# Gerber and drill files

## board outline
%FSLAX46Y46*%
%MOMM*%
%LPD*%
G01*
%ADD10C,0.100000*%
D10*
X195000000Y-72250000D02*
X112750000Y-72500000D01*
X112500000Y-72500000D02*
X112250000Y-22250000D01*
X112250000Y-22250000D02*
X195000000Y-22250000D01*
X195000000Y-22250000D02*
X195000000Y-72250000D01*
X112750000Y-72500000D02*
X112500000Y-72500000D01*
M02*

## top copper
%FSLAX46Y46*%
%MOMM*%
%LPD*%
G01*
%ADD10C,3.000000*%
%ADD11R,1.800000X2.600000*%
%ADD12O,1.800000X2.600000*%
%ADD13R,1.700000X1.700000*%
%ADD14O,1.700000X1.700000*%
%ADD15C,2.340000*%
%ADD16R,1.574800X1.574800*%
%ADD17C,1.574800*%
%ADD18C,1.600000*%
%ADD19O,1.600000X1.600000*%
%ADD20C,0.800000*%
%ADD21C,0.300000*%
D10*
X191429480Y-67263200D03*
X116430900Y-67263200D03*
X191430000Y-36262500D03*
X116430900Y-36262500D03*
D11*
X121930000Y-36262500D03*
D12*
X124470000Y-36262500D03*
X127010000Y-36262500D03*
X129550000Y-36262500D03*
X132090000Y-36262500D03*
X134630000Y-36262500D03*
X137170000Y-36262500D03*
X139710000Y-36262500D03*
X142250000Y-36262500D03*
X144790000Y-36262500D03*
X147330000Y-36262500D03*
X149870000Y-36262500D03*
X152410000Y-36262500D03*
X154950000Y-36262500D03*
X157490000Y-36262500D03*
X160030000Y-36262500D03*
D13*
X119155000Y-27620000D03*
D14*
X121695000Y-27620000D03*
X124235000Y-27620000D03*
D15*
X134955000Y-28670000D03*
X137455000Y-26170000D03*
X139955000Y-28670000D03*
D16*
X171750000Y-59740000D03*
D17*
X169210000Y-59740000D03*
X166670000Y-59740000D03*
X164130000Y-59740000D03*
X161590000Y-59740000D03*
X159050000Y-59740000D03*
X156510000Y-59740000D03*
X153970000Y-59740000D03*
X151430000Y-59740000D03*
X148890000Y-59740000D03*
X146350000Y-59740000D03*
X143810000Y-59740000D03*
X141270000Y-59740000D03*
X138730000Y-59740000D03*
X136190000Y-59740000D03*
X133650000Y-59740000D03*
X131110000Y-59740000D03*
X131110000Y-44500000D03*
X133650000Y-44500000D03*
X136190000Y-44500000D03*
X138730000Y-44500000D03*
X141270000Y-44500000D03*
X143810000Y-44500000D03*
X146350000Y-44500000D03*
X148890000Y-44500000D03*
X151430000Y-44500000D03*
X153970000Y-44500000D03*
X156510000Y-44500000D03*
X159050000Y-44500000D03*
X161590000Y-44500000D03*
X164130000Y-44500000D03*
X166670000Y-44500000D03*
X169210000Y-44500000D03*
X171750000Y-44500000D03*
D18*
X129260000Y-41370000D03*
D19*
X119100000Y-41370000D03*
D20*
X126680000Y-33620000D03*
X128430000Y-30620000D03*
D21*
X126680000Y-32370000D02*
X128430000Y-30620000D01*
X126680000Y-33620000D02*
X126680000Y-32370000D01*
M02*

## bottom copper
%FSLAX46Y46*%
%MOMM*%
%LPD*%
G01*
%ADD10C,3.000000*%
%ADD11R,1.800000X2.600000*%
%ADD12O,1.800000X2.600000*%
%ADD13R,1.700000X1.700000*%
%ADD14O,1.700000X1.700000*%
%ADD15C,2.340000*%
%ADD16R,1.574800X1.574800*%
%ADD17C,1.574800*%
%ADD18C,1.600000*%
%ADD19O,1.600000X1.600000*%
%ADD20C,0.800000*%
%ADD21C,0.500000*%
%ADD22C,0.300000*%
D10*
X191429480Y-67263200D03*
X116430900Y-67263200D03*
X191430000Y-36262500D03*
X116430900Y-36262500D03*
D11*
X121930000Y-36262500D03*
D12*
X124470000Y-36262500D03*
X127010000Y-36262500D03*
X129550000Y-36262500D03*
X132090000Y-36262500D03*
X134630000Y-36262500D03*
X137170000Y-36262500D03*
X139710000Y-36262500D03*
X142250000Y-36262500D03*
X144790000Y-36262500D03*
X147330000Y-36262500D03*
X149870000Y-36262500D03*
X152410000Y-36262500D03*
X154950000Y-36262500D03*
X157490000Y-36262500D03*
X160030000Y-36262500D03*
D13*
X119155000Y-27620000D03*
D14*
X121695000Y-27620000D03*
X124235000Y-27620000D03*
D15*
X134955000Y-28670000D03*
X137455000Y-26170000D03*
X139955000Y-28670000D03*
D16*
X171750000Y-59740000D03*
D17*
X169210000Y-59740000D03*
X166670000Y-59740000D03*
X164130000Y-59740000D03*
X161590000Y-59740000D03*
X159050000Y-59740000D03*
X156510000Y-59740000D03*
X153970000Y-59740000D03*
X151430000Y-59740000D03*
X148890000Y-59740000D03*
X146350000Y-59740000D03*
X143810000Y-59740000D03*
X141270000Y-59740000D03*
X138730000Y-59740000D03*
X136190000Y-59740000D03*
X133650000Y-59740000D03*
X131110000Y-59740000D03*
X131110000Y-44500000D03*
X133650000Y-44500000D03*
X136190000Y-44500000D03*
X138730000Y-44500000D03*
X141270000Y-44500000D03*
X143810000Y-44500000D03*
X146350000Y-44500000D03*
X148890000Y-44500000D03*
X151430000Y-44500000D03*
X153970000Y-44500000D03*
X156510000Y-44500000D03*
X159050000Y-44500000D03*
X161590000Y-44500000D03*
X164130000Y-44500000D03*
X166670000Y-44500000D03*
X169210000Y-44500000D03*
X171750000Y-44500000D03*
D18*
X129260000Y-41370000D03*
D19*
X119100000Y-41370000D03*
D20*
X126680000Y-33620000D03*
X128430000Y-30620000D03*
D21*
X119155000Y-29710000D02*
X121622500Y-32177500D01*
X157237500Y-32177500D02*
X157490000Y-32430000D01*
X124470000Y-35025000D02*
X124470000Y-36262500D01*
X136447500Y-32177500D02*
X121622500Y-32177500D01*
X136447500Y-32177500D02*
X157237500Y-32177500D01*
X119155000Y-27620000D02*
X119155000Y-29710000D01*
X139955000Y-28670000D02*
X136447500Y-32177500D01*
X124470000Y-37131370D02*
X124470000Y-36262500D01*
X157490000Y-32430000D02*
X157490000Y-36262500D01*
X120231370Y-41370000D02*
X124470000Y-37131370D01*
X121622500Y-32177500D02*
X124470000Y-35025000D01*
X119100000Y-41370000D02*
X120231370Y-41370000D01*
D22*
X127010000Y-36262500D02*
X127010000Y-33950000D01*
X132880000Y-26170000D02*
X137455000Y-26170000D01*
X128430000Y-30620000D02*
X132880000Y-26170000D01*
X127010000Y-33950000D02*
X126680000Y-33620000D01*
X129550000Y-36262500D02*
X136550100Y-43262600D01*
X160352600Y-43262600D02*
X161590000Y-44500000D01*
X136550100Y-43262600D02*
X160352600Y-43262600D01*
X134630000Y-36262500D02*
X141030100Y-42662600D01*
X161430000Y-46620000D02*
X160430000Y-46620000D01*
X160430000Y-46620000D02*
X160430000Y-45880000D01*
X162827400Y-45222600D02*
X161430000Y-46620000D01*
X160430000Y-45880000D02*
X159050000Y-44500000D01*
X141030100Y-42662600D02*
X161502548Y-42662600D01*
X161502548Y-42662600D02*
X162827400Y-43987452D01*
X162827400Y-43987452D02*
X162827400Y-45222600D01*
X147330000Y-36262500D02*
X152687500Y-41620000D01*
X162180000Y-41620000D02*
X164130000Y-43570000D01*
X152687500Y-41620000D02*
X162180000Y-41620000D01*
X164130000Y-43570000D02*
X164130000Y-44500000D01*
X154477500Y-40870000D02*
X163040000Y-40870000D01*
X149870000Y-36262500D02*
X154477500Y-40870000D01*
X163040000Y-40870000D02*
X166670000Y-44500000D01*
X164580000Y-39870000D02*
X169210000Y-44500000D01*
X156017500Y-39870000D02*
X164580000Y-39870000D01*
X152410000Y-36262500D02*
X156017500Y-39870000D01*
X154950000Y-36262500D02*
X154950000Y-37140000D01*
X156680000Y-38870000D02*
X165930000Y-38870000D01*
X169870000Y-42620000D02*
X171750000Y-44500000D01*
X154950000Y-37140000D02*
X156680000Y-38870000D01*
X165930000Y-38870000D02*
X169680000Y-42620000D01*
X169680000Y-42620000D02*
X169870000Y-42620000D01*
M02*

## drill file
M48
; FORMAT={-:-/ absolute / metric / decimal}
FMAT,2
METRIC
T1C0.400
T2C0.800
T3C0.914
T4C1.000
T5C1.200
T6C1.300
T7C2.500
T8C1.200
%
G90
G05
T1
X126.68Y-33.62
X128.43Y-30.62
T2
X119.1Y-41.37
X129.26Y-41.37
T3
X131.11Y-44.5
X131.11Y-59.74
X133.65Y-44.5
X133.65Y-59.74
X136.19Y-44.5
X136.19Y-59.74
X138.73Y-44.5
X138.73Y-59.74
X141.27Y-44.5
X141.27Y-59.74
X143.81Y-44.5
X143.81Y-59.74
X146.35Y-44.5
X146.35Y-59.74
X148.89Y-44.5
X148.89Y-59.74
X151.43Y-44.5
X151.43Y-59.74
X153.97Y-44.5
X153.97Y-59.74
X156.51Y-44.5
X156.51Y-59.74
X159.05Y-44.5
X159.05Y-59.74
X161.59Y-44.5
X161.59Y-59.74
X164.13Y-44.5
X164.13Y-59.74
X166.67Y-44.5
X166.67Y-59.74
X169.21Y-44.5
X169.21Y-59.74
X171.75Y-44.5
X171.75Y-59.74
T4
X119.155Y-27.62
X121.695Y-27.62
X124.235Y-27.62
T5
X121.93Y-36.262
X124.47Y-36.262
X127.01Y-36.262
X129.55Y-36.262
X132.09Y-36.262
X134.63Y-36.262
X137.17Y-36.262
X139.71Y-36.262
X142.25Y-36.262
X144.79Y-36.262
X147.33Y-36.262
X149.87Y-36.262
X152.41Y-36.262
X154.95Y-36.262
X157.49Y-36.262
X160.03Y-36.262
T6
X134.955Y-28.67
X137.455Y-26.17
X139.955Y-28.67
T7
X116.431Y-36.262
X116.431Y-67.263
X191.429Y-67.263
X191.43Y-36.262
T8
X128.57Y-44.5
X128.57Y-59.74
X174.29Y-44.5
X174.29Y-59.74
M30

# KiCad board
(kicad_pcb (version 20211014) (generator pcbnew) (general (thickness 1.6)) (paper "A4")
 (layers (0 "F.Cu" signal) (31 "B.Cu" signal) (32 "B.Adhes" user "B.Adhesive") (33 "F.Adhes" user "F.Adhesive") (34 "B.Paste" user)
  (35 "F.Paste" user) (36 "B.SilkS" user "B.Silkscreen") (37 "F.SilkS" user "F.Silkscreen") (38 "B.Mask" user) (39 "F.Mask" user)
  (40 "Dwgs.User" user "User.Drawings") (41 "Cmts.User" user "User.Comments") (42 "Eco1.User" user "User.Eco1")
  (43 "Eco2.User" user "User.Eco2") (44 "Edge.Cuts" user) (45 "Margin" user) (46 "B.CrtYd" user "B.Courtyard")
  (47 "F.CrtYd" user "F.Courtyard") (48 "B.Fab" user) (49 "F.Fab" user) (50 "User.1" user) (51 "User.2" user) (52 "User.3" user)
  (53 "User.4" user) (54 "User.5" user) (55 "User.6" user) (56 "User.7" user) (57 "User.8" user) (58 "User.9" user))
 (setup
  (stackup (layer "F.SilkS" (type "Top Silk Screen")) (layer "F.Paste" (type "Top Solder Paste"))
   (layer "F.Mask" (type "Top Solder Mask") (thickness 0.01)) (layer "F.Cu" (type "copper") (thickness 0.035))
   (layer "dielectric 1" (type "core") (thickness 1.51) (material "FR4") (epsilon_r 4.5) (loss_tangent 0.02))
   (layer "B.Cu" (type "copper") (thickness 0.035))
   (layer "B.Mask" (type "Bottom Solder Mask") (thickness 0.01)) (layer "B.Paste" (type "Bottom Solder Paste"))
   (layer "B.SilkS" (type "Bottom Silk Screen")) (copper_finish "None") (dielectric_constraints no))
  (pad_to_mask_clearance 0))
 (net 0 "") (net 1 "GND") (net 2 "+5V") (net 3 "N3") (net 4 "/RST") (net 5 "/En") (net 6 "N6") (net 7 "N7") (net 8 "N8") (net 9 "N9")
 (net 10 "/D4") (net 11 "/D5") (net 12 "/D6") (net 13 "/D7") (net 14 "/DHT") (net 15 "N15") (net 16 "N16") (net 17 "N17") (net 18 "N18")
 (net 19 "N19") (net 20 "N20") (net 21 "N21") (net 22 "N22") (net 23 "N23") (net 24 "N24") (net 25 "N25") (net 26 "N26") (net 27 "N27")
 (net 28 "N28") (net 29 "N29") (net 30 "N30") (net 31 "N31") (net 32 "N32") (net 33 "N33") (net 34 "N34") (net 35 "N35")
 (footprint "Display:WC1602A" (layer "F.Cu") (at 121.93 36.2625)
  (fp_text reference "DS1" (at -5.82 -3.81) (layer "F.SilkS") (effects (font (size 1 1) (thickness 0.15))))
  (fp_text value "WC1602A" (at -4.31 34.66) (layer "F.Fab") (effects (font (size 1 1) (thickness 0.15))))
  (pad "" thru_hole circle (at 69.49948 31.0007) (size 3 3) (drill 2.5) (layers *.Cu *.Mask))
  (pad "" thru_hole circle (at -5.4991 31.0007) (size 3 3) (drill 2.5) (layers *.Cu *.Mask))
  (pad "" thru_hole circle (at 69.5 0) (size 3 3) (drill 2.5) (layers *.Cu *.Mask))
  (pad "" thru_hole circle (at -5.4991 0) (size 3 3) (drill 2.5) (layers *.Cu *.Mask))
  (pad "1" thru_hole rect (at 0 0) (size 1.8 2.6) (drill 1.2) (layers *.Cu *.Mask) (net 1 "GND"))
  (pad "2" thru_hole oval (at 2.54 0) (size 1.8 2.6) (drill 1.2) (layers *.Cu *.Mask) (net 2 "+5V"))
  (pad "3" thru_hole oval (at 5.08 0) (size 1.8 2.6) (drill 1.2) (layers *.Cu *.Mask) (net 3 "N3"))
  (pad "4" thru_hole oval (at 7.62 0) (size 1.8 2.6) (drill 1.2) (layers *.Cu *.Mask) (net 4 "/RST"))
  (pad "5" thru_hole oval (at 10.16 0) (size 1.8 2.6) (drill 1.2) (layers *.Cu *.Mask) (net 1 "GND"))
  (pad "6" thru_hole oval (at 12.7 0) (size 1.8 2.6) (drill 1.2) (layers *.Cu *.Mask) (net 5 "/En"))
  (pad "7" thru_hole oval (at 15.24 0) (size 1.8 2.6) (drill 1.2) (layers *.Cu *.Mask) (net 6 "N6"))
  (pad "8" thru_hole oval (at 17.78 0) (size 1.8 2.6) (drill 1.2) (layers *.Cu *.Mask) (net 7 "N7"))
  (pad "9" thru_hole oval (at 20.32 0) (size 1.8 2.6) (drill 1.2) (layers *.Cu *.Mask) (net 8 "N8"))
  (pad "10" thru_hole oval (at 22.86 0) (size 1.8 2.6) (drill 1.2) (layers *.Cu *.Mask) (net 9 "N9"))
  (pad "11" thru_hole oval (at 25.4 0) (size 1.8 2.6) (drill 1.2) (layers *.Cu *.Mask) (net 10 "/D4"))
  (pad "12" thru_hole oval (at 27.94 0) (size 1.8 2.6) (drill 1.2) (layers *.Cu *.Mask) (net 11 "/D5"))
  (pad "13" thru_hole oval (at 30.48 0) (size 1.8 2.6) (drill 1.2) (layers *.Cu *.Mask) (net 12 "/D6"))
  (pad "14" thru_hole oval (at 33.02 0) (size 1.8 2.6) (drill 1.2) (layers *.Cu *.Mask) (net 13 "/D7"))
  (pad "15" thru_hole oval (at 35.56 0) (size 1.8 2.6) (drill 1.2) (layers *.Cu *.Mask) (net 2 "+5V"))
  (pad "16" thru_hole oval (at 38.1 0) (size 1.8 2.6) (drill 1.2) (layers *.Cu *.Mask) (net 1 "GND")))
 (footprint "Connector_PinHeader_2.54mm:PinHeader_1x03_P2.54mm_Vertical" (layer "F.Cu") (at 119.155 27.62 90)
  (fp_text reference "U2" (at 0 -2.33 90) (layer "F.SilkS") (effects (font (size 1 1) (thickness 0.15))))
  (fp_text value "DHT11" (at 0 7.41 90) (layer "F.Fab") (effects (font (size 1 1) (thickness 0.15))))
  (pad "1" thru_hole rect (at 0 0 90) (size 1.7 1.7) (drill 1) (layers *.Cu *.Mask) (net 2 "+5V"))
  (pad "2" thru_hole oval (at 0 2.54 90) (size 1.7 1.7) (drill 1) (layers *.Cu *.Mask) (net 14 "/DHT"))
  (pad "3" thru_hole oval (at 0 5.08 90) (size 1.7 1.7) (drill 1) (layers *.Cu *.Mask) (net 1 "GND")))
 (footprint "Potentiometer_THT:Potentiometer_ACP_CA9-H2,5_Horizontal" (layer "F.Cu") (at 134.955 28.67 90)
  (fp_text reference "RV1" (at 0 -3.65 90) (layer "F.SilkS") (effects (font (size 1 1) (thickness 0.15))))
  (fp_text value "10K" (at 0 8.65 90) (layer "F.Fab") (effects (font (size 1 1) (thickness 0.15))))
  (pad "1" thru_hole circle (at 0 0 90) (size 2.34 2.34) (drill 1.3) (layers *.Cu *.Mask) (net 1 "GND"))
  (pad "2" thru_hole circle (at 2.5 2.5 90) (size 2.34 2.34) (drill 1.3) (layers *.Cu *.Mask) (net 3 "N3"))
  (pad "3" thru_hole circle (at 0 5 90) (size 2.34 2.34) (drill 1.3) (layers *.Cu *.Mask) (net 2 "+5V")))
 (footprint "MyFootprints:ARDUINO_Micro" (layer "B.Cu") (at 151.43 52.12 90)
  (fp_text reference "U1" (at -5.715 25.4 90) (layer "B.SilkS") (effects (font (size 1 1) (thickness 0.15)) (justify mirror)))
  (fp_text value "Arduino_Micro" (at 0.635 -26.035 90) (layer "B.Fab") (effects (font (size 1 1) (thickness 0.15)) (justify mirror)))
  (pad "" np_thru_hole circle (at -7.62 -22.86 90) (size 1.2 1.2) (drill 1.2) (layers *.Cu *.Mask))
  (pad "" np_thru_hole circle (at 7.62 22.86 90) (size 1.2 1.2) (drill 1.2) (layers *.Cu *.Mask))
  (pad "" np_thru_hole circle (at -7.62 22.86 90) (size 1.2 1.2) (drill 1.2) (layers *.Cu *.Mask))
  (pad "" np_thru_hole circle (at 7.62 -22.86 90) (size 1.2 1.2) (drill 1.2) (layers *.Cu *.Mask))
  (pad "1" thru_hole rect (at -7.62 20.32 90) (size 1.5748 1.5748) (drill 0.9144) (layers *.Cu *.Mask) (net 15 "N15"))
  (pad "2" thru_hole circle (at -7.62 17.78 90) (size 1.5748 1.5748) (drill 0.9144) (layers *.Cu *.Mask) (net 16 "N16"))
  (pad "3" thru_hole circle (at -7.62 15.24 90) (size 1.5748 1.5748) (drill 0.9144) (layers *.Cu *.Mask) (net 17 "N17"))
  (pad "4" thru_hole circle (at -7.62 12.7 90) (size 1.5748 1.5748) (drill 0.9144) (layers *.Cu *.Mask) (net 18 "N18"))
  (pad "5" thru_hole circle (at -7.62 10.16 90) (size 1.5748 1.5748) (drill 0.9144) (layers *.Cu *.Mask) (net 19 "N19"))
  (pad "6" thru_hole circle (at -7.62 7.62 90) (size 1.5748 1.5748) (drill 0.9144) (layers *.Cu *.Mask) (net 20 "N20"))
  (pad "7" thru_hole circle (at -7.62 5.08 90) (size 1.5748 1.5748) (drill 0.9144) (layers *.Cu *.Mask) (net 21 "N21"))
  (pad "8" thru_hole circle (at -7.62 2.54 90) (size 1.5748 1.5748) (drill 0.9144) (layers *.Cu *.Mask) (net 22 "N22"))
  (pad "9" thru_hole circle (at -7.62 0 90) (size 1.5748 1.5748) (drill 0.9144) (layers *.Cu *.Mask) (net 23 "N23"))
  (pad "10" thru_hole circle (at -7.62 -2.54 90) (size 1.5748 1.5748) (drill 0.9144) (layers *.Cu *.Mask))
  (pad "11" thru_hole circle (at -7.62 -5.08 90) (size 1.5748 1.5748) (drill 0.9144) (layers *.Cu *.Mask))
  (pad "12" thru_hole circle (at -7.62 -7.62 90) (size 1.5748 1.5748) (drill 0.9144) (layers *.Cu *.Mask) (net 2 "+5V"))
  (pad "13" thru_hole circle (at -7.62 -10.16 90) (size 1.5748 1.5748) (drill 0.9144) (layers *.Cu *.Mask) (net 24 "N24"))
  (pad "14" thru_hole circle (at -7.62 -12.7 90) (size 1.5748 1.5748) (drill 0.9144) (layers *.Cu *.Mask) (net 1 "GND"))
  (pad "15" thru_hole circle (at -7.62 -15.24 90) (size 1.5748 1.5748) (drill 0.9144) (layers *.Cu *.Mask) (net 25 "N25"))
  (pad "16" thru_hole circle (at -7.62 -17.78 90) (size 1.5748 1.5748) (drill 0.9144) (layers *.Cu *.Mask) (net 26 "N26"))
  (pad "17" thru_hole circle (at -7.62 -20.32 90) (size 1.5748 1.5748) (drill 0.9144) (layers *.Cu *.Mask) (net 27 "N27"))
  (pad "18" thru_hole circle (at 7.62 -20.32 90) (size 1.5748 1.5748) (drill 0.9144) (layers *.Cu *.Mask) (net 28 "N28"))
  (pad "19" thru_hole circle (at 7.62 -17.78 90) (size 1.5748 1.5748) (drill 0.9144) (layers *.Cu *.Mask) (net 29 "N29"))
  (pad "20" thru_hole circle (at 7.62 -15.24 90) (size 1.5748 1.5748) (drill 0.9144) (layers *.Cu *.Mask) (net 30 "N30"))
  (pad "21" thru_hole circle (at 7.62 -12.7 90) (size 1.5748 1.5748) (drill 0.9144) (layers *.Cu *.Mask) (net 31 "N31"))
  (pad "22" thru_hole circle (at 7.62 -10.16 90) (size 1.5748 1.5748) (drill 0.9144) (layers *.Cu *.Mask))
  (pad "23" thru_hole circle (at 7.62 -7.62 90) (size 1.5748 1.5748) (drill 0.9144) (layers *.Cu *.Mask) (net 1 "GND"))
  (pad "24" thru_hole circle (at 7.62 -5.08 90) (size 1.5748 1.5748) (drill 0.9144) (layers *.Cu *.Mask) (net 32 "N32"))
  (pad "25" thru_hole circle (at 7.62 -2.54 90) (size 1.5748 1.5748) (drill 0.9144) (layers *.Cu *.Mask) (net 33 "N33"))
  (pad "26" thru_hole circle (at 7.62 0 90) (size 1.5748 1.5748) (drill 0.9144) (layers *.Cu *.Mask) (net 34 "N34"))
  (pad "27" thru_hole circle (at 7.62 2.54 90) (size 1.5748 1.5748) (drill 0.9144) (layers *.Cu *.Mask) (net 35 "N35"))
  (pad "28" thru_hole circle (at 7.62 5.08 90) (size 1.5748 1.5748) (drill 0.9144) (layers *.Cu *.Mask) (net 14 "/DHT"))
  (pad "29" thru_hole circle (at 7.62 7.62 90) (size 1.5748 1.5748) (drill 0.9144) (layers *.Cu *.Mask) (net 5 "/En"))
  (pad "30" thru_hole circle (at 7.62 10.16 90) (size 1.5748 1.5748) (drill 0.9144) (layers *.Cu *.Mask) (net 4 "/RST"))
  (pad "31" thru_hole circle (at 7.62 12.7 90) (size 1.5748 1.5748) (drill 0.9144) (layers *.Cu *.Mask) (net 10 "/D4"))
  (pad "32" thru_hole circle (at 7.62 15.24 90) (size 1.5748 1.5748) (drill 0.9144) (layers *.Cu *.Mask) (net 11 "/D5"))
  (pad "33" thru_hole circle (at 7.62 17.78 90) (size 1.5748 1.5748) (drill 0.9144) (layers *.Cu *.Mask) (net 12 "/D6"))
  (pad "34" thru_hole circle (at 7.62 20.32 90) (size 1.5748 1.5748) (drill 0.9144) (layers *.Cu *.Mask) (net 13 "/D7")))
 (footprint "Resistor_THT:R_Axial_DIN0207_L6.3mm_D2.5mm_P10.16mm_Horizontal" (layer "B.Cu") (at 129.26 41.37 180)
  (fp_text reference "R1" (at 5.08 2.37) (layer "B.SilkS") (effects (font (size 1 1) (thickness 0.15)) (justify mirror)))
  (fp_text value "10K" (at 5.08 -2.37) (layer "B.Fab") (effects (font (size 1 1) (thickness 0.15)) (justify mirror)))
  (pad "1" thru_hole circle (at 0 0 180) (size 1.6 1.6) (drill 0.8) (layers *.Cu *.Mask) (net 14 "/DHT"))
  (pad "2" thru_hole oval (at 10.16 0 180) (size 1.6 1.6) (drill 0.8) (layers *.Cu *.Mask) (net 2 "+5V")))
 (gr_line (start 195 72.25) (end 112.75 72.5) (layer "Edge.Cuts") (width 0.1))
 (gr_line (start 112.5 72.5) (end 112.25 22.25) (layer "Edge.Cuts") (width 0.1))
 (gr_line (start 112.25 22.25) (end 195 22.25) (layer "Edge.Cuts") (width 0.1))
 (gr_line (start 195 22.25) (end 195 72.25) (layer "Edge.Cuts") (width 0.1))
 (gr_line (start 112.75 72.5) (end 112.5 72.5) (layer "Edge.Cuts") (width 0.1))
 (segment (start 119.155 29.71) (end 121.6225 32.1775) (width 0.5) (layer "B.Cu") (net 2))
 (segment (start 157.2375 32.1775) (end 157.49 32.43) (width 0.5) (layer "B.Cu") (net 2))
 (segment (start 124.47 35.025) (end 124.47 36.2625) (width 0.5) (layer "B.Cu") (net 2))
 (segment (start 136.4475 32.1775) (end 121.6225 32.1775) (width 0.5) (layer "B.Cu") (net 2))
 (segment (start 136.4475 32.1775) (end 157.2375 32.1775) (width 0.5) (layer "B.Cu") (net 2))
 (segment (start 119.155 27.62) (end 119.155 29.71) (width 0.5) (layer "B.Cu") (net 2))
 (segment (start 139.955 28.67) (end 136.4475 32.1775) (width 0.5) (layer "B.Cu") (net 2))
 (segment (start 124.47 37.13137) (end 124.47 36.2625) (width 0.5) (layer "B.Cu") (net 2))
 (segment (start 157.49 32.43) (end 157.49 36.2625) (width 0.5) (layer "B.Cu") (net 2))
 (segment (start 120.23137 41.37) (end 124.47 37.13137) (width 0.5) (layer "B.Cu") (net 2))
 (segment (start 121.6225 32.1775) (end 124.47 35.025) (width 0.5) (layer "B.Cu") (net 2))
 (segment (start 119.1 41.37) (end 120.23137 41.37) (width 0.5) (layer "B.Cu") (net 2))
 (segment (start 126.68 32.37) (end 128.43 30.62) (width 0.3) (layer "F.Cu") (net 3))
 (segment (start 126.68 33.62) (end 126.68 32.37) (width 0.3) (layer "F.Cu") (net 3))
 (via (at 126.68 33.62) (size 0.8) (drill 0.4) (layers "F.Cu" "B.Cu") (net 3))
 (via (at 128.43 30.62) (size 0.8) (drill 0.4) (layers "F.Cu" "B.Cu") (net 3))
 (segment (start 127.01 36.2625) (end 127.01 33.95) (width 0.3) (layer "B.Cu") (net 3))
 (segment (start 132.88 26.17) (end 137.455 26.17) (width 0.3) (layer "B.Cu") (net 3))
 (segment (start 128.43 30.62) (end 132.88 26.17) (width 0.3) (layer "B.Cu") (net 3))
 (segment (start 127.01 33.95) (end 126.68 33.62) (width 0.3) (layer "B.Cu") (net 3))
 (segment (start 129.55 36.2625) (end 136.5501 43.2626) (width 0.3) (layer "B.Cu") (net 4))
 (segment (start 160.3526 43.2626) (end 161.59 44.5) (width 0.3) (layer "B.Cu") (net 4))
 (segment (start 136.5501 43.2626) (end 160.3526 43.2626) (width 0.3) (layer "B.Cu") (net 4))
 (segment (start 134.63 36.2625) (end 141.0301 42.6626) (width 0.3) (layer "B.Cu") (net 5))
 (segment (start 161.43 46.62) (end 160.43 46.62) (width 0.3) (layer "B.Cu") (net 5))
 (segment (start 160.43 46.62) (end 160.43 45.88) (width 0.3) (layer "B.Cu") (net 5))
 (segment (start 162.8274 45.2226) (end 161.43 46.62) (width 0.3) (layer "B.Cu") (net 5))
 (segment (start 160.43 45.88) (end 159.05 44.5) (width 0.3) (layer "B.Cu") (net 5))
 (segment (start 141.0301 42.6626) (end 161.502548 42.6626) (width 0.3) (layer "B.Cu") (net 5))
 (segment (start 161.502548 42.6626) (end 162.8274 43.987452) (width 0.3) (layer "B.Cu") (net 5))
 (segment (start 162.8274 43.987452) (end 162.8274 45.2226) (width 0.3) (layer "B.Cu") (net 5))
 (segment (start 147.33 36.2625) (end 152.6875 41.62) (width 0.3) (layer "B.Cu") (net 10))
 (segment (start 162.18 41.62) (end 164.13 43.57) (width 0.3) (layer "B.Cu") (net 10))
 (segment (start 152.6875 41.62) (end 162.18 41.62) (width 0.3) (layer "B.Cu") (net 10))
 (segment (start 164.13 43.57) (end 164.13 44.5) (width 0.3) (layer "B.Cu") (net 10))
 (segment (start 154.4775 40.87) (end 163.04 40.87) (width 0.3) (layer "B.Cu") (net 11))
 (segment (start 149.87 36.2625) (end 154.4775 40.87) (width 0.3) (layer "B.Cu") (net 11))
 (segment (start 163.04 40.87) (end 166.67 44.5) (width 0.3) (layer "B.Cu") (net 11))
 (segment (start 164.58 39.87) (end 169.21 44.5) (width 0.3) (layer "B.Cu") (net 12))
 (segment (start 156.0175 39.87) (end 164.58 39.87) (width 0.3) (layer "B.Cu") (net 12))
 (segment (start 152.41 36.2625) (end 156.0175 39.87) (width 0.3) (layer "B.Cu") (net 12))
 (segment (start 154.95 36.2625) (end 154.95 37.14) (width 0.3) (layer "B.Cu") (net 13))
 (segment (start 156.68 38.87) (end 165.93 38.87) (width 0.3) (layer "B.Cu") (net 13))
 (segment (start 169.87 42.62) (end 171.75 44.5) (width 0.3) (layer "B.Cu") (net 13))
 (segment (start 154.95 37.14) (end 156.68 38.87) (width 0.3) (layer "B.Cu") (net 13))
 (segment (start 165.93 38.87) (end 169.68 42.62) (width 0.3) (layer "B.Cu") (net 13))
 (segment (start 169.68 42.62) (end 169.87 42.62) (width 0.3) (layer "B.Cu") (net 13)))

